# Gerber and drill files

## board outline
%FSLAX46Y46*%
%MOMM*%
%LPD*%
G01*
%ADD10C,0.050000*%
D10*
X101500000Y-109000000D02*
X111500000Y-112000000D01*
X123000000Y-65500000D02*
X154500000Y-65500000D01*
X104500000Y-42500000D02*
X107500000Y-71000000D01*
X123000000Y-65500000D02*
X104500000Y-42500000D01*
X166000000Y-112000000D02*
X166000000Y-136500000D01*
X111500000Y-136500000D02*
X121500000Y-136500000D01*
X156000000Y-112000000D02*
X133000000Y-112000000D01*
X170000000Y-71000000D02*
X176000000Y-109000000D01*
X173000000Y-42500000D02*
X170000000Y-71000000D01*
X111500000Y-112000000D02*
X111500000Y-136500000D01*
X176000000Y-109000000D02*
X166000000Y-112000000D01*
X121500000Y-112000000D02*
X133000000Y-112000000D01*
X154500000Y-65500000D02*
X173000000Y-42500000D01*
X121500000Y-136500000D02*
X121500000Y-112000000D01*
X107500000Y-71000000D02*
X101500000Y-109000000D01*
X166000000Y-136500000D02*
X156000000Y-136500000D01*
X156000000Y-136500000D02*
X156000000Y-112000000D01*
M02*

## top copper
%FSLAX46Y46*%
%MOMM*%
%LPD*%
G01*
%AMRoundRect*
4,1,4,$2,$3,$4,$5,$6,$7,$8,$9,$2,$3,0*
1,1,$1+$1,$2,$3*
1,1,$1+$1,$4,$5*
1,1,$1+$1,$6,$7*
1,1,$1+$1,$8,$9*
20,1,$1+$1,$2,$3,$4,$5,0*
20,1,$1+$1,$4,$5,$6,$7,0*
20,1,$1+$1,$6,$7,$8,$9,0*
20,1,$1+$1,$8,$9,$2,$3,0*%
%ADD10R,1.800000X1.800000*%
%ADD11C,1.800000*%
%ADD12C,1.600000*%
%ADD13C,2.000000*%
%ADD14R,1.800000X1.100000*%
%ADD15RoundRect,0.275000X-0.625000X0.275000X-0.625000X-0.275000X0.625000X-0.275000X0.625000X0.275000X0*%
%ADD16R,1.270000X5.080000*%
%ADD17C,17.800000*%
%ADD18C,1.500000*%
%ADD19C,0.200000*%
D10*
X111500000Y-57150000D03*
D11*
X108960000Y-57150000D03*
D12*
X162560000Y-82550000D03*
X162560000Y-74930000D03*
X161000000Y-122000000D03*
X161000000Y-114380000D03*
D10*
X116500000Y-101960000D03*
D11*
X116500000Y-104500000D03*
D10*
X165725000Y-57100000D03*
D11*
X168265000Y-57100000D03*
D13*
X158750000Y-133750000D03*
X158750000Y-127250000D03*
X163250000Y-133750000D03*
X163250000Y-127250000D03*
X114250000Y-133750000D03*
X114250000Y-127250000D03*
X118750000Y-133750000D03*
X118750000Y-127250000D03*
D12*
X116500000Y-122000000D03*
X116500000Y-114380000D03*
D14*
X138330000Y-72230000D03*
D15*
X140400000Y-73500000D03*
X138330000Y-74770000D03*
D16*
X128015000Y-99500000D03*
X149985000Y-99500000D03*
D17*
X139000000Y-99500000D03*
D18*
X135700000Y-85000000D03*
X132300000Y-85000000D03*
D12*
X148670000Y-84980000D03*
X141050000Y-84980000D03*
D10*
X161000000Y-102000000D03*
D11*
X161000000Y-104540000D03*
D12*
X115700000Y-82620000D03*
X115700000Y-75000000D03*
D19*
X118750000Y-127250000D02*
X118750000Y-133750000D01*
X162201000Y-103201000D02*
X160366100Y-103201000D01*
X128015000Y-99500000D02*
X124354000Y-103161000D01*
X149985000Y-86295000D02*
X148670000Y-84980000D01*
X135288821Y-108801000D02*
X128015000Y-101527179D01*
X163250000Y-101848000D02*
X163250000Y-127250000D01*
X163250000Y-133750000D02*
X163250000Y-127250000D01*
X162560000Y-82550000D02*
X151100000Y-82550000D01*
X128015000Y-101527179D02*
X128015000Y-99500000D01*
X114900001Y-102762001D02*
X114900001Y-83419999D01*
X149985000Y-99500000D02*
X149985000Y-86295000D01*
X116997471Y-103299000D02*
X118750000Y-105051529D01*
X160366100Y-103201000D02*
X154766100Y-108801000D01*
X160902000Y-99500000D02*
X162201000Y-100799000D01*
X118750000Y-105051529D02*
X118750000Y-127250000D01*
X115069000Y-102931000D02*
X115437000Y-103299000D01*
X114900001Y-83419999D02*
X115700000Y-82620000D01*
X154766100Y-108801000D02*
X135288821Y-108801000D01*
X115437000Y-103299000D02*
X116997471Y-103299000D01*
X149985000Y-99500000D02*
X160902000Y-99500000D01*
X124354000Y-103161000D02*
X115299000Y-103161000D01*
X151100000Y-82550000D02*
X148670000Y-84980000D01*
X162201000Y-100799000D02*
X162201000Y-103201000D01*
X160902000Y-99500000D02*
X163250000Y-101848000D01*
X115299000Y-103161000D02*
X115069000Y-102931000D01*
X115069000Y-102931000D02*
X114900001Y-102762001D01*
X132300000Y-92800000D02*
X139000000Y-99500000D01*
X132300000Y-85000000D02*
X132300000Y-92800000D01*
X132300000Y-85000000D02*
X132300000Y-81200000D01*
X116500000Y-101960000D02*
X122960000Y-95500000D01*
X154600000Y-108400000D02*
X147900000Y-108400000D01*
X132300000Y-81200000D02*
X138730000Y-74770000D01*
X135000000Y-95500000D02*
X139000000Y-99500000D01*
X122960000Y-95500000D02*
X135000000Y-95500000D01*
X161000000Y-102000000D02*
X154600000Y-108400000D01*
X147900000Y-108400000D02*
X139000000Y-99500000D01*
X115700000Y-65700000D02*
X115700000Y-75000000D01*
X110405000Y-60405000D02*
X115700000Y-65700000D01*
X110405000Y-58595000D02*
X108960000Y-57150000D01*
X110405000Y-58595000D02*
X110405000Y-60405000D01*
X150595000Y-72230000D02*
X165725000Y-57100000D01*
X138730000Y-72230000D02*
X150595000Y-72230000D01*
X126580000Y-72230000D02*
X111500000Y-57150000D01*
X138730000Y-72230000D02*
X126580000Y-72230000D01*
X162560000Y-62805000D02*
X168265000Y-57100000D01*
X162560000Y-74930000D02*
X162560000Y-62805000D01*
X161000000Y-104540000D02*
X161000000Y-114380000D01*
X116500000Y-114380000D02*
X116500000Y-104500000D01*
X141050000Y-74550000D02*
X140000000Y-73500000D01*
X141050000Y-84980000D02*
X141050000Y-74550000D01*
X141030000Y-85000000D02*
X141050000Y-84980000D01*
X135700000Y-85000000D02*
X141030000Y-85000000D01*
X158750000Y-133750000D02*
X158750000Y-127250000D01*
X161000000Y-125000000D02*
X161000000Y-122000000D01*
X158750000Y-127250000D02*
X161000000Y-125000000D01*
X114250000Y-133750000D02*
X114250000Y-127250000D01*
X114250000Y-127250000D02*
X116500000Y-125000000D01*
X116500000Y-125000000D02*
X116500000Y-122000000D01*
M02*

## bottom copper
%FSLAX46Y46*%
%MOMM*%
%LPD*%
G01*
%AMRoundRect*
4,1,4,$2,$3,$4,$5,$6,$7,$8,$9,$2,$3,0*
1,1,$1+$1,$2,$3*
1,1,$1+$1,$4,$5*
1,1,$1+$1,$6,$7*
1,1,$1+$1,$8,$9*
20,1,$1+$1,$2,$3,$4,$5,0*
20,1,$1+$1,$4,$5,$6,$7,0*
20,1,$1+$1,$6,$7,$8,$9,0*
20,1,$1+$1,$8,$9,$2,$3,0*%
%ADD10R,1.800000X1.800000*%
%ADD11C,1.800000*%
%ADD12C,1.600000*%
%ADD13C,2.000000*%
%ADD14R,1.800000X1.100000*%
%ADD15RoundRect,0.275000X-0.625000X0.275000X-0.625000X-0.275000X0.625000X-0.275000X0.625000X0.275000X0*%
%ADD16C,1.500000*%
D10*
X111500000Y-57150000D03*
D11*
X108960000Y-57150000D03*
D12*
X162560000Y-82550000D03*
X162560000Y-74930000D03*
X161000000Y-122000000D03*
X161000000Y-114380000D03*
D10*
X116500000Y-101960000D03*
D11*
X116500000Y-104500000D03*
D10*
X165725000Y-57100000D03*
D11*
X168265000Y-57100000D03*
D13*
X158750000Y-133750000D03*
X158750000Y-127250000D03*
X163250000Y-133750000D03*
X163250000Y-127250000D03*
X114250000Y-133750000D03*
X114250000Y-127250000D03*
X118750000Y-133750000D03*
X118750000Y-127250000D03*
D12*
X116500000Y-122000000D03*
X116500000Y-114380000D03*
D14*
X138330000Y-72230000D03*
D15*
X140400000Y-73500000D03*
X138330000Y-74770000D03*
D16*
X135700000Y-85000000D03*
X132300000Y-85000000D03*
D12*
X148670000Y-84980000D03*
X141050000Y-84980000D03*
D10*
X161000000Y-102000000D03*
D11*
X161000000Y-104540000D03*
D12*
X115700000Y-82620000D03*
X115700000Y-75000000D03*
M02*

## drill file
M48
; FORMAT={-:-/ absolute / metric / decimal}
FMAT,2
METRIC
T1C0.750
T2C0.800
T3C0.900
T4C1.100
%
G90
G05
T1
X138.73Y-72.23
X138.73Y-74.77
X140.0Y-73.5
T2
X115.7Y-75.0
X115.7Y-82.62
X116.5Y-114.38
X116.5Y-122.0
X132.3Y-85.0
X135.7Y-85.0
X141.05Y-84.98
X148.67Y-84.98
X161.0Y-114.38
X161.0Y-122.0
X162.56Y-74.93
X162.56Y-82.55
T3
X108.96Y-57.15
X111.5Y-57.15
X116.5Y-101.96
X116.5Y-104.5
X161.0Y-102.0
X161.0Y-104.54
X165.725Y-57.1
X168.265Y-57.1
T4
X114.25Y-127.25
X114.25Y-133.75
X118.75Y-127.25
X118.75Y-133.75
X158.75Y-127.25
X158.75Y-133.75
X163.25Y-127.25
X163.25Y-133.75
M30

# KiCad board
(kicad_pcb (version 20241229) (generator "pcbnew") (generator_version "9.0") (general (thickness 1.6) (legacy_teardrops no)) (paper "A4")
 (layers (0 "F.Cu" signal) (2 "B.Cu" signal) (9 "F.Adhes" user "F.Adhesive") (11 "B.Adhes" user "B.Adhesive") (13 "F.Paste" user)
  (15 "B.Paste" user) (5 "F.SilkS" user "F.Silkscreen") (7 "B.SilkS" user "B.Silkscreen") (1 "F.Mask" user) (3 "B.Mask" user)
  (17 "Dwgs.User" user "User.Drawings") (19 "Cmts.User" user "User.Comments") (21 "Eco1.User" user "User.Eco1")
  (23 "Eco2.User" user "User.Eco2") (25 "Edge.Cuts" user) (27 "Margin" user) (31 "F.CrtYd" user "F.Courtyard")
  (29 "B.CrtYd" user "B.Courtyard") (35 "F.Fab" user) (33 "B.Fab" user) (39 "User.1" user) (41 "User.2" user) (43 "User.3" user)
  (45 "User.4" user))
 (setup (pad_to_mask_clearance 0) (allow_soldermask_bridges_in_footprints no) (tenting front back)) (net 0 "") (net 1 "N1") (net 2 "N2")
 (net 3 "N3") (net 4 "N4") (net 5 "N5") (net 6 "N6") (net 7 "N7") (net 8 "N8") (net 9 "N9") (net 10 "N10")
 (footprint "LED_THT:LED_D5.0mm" (layer "F.Cu") (at 111.5 57.15 180)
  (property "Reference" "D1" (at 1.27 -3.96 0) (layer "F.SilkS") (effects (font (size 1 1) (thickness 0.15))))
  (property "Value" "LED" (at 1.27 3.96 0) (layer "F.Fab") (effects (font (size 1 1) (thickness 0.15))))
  (pad "1" thru_hole rect (at 0 0 180) (size 1.8 1.8) (drill 0.9) (layers "*.Cu" "*.Mask") (remove_unused_layers no) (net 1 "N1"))
  (pad "2" thru_hole circle (at 2.54 0 180) (size 1.8 1.8) (drill 0.9) (layers "*.Cu" "*.Mask") (remove_unused_layers no) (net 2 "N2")))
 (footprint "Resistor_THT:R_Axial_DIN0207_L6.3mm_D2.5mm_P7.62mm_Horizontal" (layer "F.Cu") (at 162.56 82.55 90)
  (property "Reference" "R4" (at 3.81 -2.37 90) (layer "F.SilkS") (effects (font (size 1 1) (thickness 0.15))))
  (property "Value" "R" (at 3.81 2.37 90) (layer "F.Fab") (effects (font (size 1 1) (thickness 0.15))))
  (pad "1" thru_hole circle (at 0 0 90) (size 1.6 1.6) (drill 0.8) (layers "*.Cu" "*.Mask") (remove_unused_layers no) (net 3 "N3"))
  (pad "2" thru_hole circle (at 7.62 0 90) (size 1.6 1.6) (drill 0.8) (layers "*.Cu" "*.Mask") (remove_unused_layers no) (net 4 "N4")))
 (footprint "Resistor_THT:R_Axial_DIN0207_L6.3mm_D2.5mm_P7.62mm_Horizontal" (layer "F.Cu") (at 161 122 90)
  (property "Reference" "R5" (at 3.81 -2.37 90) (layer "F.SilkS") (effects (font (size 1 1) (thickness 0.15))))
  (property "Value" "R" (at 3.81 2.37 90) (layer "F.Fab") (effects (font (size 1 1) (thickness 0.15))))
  (pad "1" thru_hole circle (at 0 0 90) (size 1.6 1.6) (drill 0.8) (layers "*.Cu" "*.Mask") (remove_unused_layers no) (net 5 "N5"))
  (pad "2" thru_hole circle (at 7.62 0 90) (size 1.6 1.6) (drill 0.8) (layers "*.Cu" "*.Mask") (remove_unused_layers no) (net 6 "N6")))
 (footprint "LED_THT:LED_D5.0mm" (layer "F.Cu") (at 116.5 101.96 -90)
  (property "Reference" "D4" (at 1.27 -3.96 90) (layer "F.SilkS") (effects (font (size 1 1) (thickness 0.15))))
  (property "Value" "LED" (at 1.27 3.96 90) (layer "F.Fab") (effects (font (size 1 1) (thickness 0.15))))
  (pad "1" thru_hole rect (at 0 0 270) (size 1.8 1.8) (drill 0.9) (layers "*.Cu" "*.Mask") (remove_unused_layers no) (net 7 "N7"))
  (pad "2" thru_hole circle (at 2.54 0 270) (size 1.8 1.8) (drill 0.9) (layers "*.Cu" "*.Mask") (remove_unused_layers no) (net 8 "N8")))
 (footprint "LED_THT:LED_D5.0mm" (layer "F.Cu") (at 165.725 57.1)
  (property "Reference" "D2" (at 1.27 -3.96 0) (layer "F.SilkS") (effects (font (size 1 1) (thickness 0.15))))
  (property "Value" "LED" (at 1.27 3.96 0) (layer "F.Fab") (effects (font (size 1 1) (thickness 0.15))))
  (pad "1" thru_hole rect (at 0 0) (size 1.8 1.8) (drill 0.9) (layers "*.Cu" "*.Mask") (remove_unused_layers no) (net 1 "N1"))
  (pad "2" thru_hole circle (at 2.54 0) (size 1.8 1.8) (drill 0.9) (layers "*.Cu" "*.Mask") (remove_unused_layers no) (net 4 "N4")))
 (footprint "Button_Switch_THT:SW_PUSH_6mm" (layer "F.Cu") (at 158.75 133.75 90)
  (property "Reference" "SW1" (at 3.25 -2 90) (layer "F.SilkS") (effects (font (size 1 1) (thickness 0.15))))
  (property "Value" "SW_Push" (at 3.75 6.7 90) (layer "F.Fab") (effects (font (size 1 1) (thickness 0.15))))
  (pad "1" thru_hole circle (at 0 0 180) (size 2 2) (drill 1.1) (layers "*.Cu" "*.Mask") (remove_unused_layers no) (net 5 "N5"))
  (pad "1" thru_hole circle (at 6.5 0 180) (size 2 2) (drill 1.1) (layers "*.Cu" "*.Mask") (remove_unused_layers no) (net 5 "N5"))
  (pad "2" thru_hole circle (at 0 4.5 180) (size 2 2) (drill 1.1) (layers "*.Cu" "*.Mask") (remove_unused_layers no) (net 3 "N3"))
  (pad "2" thru_hole circle (at 6.5 4.5 180) (size 2 2) (drill 1.1) (layers "*.Cu" "*.Mask") (remove_unused_layers no) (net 3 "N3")))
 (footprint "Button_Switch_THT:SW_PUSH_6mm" (layer "F.Cu") (at 114.25 133.75 90)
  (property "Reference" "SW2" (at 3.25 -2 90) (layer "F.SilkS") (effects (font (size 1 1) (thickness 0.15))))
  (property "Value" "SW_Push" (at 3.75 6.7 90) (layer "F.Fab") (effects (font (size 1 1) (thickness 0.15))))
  (pad "1" thru_hole circle (at 0 0 180) (size 2 2) (drill 1.1) (layers "*.Cu" "*.Mask") (remove_unused_layers no) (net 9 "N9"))
  (pad "1" thru_hole circle (at 6.5 0 180) (size 2 2) (drill 1.1) (layers "*.Cu" "*.Mask") (remove_unused_layers no) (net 9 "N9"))
  (pad "2" thru_hole circle (at 0 4.5 180) (size 2 2) (drill 1.1) (layers "*.Cu" "*.Mask") (remove_unused_layers no) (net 3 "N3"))
  (pad "2" thru_hole circle (at 6.5 4.5 180) (size 2 2) (drill 1.1) (layers "*.Cu" "*.Mask") (remove_unused_layers no) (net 3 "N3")))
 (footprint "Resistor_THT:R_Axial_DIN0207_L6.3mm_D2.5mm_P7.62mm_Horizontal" (layer "F.Cu") (at 116.5 122 90)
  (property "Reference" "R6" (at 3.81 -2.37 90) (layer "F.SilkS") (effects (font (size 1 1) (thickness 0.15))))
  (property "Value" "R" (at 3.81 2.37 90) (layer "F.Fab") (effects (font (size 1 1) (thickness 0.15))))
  (pad "1" thru_hole circle (at 0 0 90) (size 1.6 1.6) (drill 0.8) (layers "*.Cu" "*.Mask") (remove_unused_layers no) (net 9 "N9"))
  (pad "2" thru_hole circle (at 7.62 0 90) (size 1.6 1.6) (drill 0.8) (layers "*.Cu" "*.Mask") (remove_unused_layers no) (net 8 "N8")))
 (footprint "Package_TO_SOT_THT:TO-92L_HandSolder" (layer "F.Cu") (at 138.73 72.23 -90)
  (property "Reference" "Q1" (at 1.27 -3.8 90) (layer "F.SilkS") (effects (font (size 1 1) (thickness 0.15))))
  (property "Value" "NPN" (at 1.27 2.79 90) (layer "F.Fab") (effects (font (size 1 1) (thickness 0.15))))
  (pad "1" thru_hole rect (at 0 0 270) (size 1.1 1.8) (drill 0.75 (offset 0 0.4)) (layers "*.Cu" "*.Mask") (remove_unused_layers no)
   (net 1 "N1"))
  (pad "2" thru_hole roundrect (at 1.27 -1.27 270) (size 1.1 1.8) (drill 0.75 (offset 0 -0.4)) (layers "*.Cu" "*.Mask")
   (remove_unused_layers no) (roundrect_rratio 0.25) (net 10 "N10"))
  (pad "3" thru_hole roundrect (at 2.54 0 270) (size 1.1 1.8) (drill 0.75 (offset 0 0.4)) (layers "*.Cu" "*.Mask") (remove_unused_layers no)
   (roundrect_rratio 0.25) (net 7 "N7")))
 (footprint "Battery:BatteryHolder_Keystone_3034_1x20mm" (layer "F.Cu") (at 139 99.5)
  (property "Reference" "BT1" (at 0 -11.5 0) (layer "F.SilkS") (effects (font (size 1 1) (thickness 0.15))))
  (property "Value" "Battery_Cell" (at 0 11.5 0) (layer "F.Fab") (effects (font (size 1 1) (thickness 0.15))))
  (pad "1" smd rect (at -10.985 0) (size 1.27 5.08) (layers "F.Cu" "F.Mask" "F.Paste") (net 3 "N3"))
  (pad "1" smd rect (at 10.985 0) (size 1.27 5.08) (layers "F.Cu" "F.Mask" "F.Paste") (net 3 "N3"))
  (pad "2" smd circle (at 0 0) (size 17.8 17.8) (layers "F.Cu" "F.Mask") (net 7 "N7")))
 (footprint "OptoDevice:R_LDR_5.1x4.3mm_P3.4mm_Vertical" (layer "F.Cu") (at 135.7 85 180)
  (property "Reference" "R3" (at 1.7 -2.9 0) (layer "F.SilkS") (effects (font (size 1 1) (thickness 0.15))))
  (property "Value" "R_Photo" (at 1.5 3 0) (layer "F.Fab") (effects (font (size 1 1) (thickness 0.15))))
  (pad "1" thru_hole circle (at 0 0 180) (size 1.5 1.5) (drill 0.8) (layers "*.Cu" "*.Mask") (remove_unused_layers no) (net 10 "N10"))
  (pad "2" thru_hole circle (at 3.4 0 180) (size 1.5 1.5) (drill 0.8) (layers "*.Cu" "*.Mask") (remove_unused_layers no) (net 7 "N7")))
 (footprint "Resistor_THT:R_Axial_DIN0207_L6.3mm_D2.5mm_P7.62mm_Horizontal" (layer "F.Cu") (at 148.67 84.98 180)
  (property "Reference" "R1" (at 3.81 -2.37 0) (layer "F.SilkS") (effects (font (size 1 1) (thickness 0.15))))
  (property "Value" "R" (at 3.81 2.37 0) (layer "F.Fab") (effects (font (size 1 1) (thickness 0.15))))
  (pad "1" thru_hole circle (at 0 0 180) (size 1.6 1.6) (drill 0.8) (layers "*.Cu" "*.Mask") (remove_unused_layers no) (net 3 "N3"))
  (pad "2" thru_hole circle (at 7.62 0 180) (size 1.6 1.6) (drill 0.8) (layers "*.Cu" "*.Mask") (remove_unused_layers no) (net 10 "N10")))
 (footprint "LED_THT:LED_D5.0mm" (layer "F.Cu") (at 161 102 -90)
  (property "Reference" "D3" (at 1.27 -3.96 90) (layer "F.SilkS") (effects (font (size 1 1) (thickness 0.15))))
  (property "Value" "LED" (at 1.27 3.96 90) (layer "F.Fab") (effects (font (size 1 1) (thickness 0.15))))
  (pad "1" thru_hole rect (at 0 0 270) (size 1.8 1.8) (drill 0.9) (layers "*.Cu" "*.Mask") (remove_unused_layers no) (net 7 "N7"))
  (pad "2" thru_hole circle (at 2.54 0 270) (size 1.8 1.8) (drill 0.9) (layers "*.Cu" "*.Mask") (remove_unused_layers no) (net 6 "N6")))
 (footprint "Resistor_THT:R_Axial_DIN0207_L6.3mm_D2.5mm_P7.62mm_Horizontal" (layer "F.Cu") (at 115.7 82.62 90)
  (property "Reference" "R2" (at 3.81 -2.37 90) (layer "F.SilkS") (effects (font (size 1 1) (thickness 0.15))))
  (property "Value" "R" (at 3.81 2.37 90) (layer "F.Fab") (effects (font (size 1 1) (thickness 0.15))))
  (pad "1" thru_hole circle (at 0 0 90) (size 1.6 1.6) (drill 0.8) (layers "*.Cu" "*.Mask") (remove_unused_layers no) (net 3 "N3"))
  (pad "2" thru_hole circle (at 7.62 0 90) (size 1.6 1.6) (drill 0.8) (layers "*.Cu" "*.Mask") (remove_unused_layers no) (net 2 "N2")))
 (gr_line (start 101.5 109) (end 111.5 112) (stroke (width 0.05) (type default)) (layer "Edge.Cuts"))
 (gr_line (start 123 65.5) (end 154.5 65.5) (stroke (width 0.05) (type default)) (layer "Edge.Cuts"))
 (gr_line (start 104.5 42.5) (end 107.5 71) (stroke (width 0.05) (type default)) (layer "Edge.Cuts"))
 (gr_line (start 123 65.5) (end 104.5 42.5) (stroke (width 0.05) (type default)) (layer "Edge.Cuts"))
 (gr_line (start 166 112) (end 166 136.5) (stroke (width 0.05) (type default)) (layer "Edge.Cuts"))
 (gr_line (start 111.5 136.5) (end 121.5 136.5) (stroke (width 0.05) (type default)) (layer "Edge.Cuts"))
 (gr_line (start 156 112) (end 133 112) (stroke (width 0.05) (type default)) (layer "Edge.Cuts"))
 (gr_line (start 170 71) (end 176 109) (stroke (width 0.05) (type default)) (layer "Edge.Cuts"))
 (gr_line (start 173 42.5) (end 170 71) (stroke (width 0.05) (type default)) (layer "Edge.Cuts"))
 (gr_line (start 111.5 112) (end 111.5 136.5) (stroke (width 0.05) (type default)) (layer "Edge.Cuts"))
 (gr_line (start 176 109) (end 166 112) (stroke (width 0.05) (type default)) (layer "Edge.Cuts"))
 (gr_line (start 121.5 112) (end 133 112) (stroke (width 0.05) (type default)) (layer "Edge.Cuts"))
 (gr_line (start 154.5 65.5) (end 173 42.5) (stroke (width 0.05) (type default)) (layer "Edge.Cuts"))
 (gr_line (start 121.5 136.5) (end 121.5 112) (stroke (width 0.05) (type default)) (layer "Edge.Cuts"))
 (gr_line (start 107.5 71) (end 101.5 109) (stroke (width 0.05) (type default)) (layer "Edge.Cuts"))
 (gr_line (start 166 136.5) (end 156 136.5) (stroke (width 0.05) (type default)) (layer "Edge.Cuts"))
 (gr_line (start 156 136.5) (end 156 112) (stroke (width 0.05) (type default)) (layer "Edge.Cuts"))
 (segment (start 118.75 127.25) (end 118.75 133.75) (width 0.2) (layer "F.Cu") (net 3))
 (segment (start 162.201 103.201) (end 160.3661 103.201) (width 0.2) (layer "F.Cu") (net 3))
 (segment (start 128.015 99.5) (end 124.354 103.161) (width 0.2) (layer "F.Cu") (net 3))
 (segment (start 149.985 86.295) (end 148.67 84.98) (width 0.2) (layer "F.Cu") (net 3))
 (segment (start 135.288821 108.801) (end 128.015 101.527179) (width 0.2) (layer "F.Cu") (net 3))
 (segment (start 163.25 101.848) (end 163.25 127.25) (width 0.2) (layer "F.Cu") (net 3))
 (segment (start 163.25 133.75) (end 163.25 127.25) (width 0.2) (layer "F.Cu") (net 3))
 (segment (start 162.56 82.55) (end 151.1 82.55) (width 0.2) (layer "F.Cu") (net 3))
 (segment (start 128.015 101.527179) (end 128.015 99.5) (width 0.2) (layer "F.Cu") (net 3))
 (segment (start 114.900001 102.762001) (end 114.900001 83.419999) (width 0.2) (layer "F.Cu") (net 3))
 (segment (start 149.985 99.5) (end 149.985 86.295) (width 0.2) (layer "F.Cu") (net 3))
 (segment (start 116.997471 103.299) (end 118.75 105.051529) (width 0.2) (layer "F.Cu") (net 3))
 (segment (start 160.3661 103.201) (end 154.7661 108.801) (width 0.2) (layer "F.Cu") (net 3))
 (segment (start 160.902 99.5) (end 162.201 100.799) (width 0.2) (layer "F.Cu") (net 3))
 (segment (start 118.75 105.051529) (end 118.75 127.25) (width 0.2) (layer "F.Cu") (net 3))
 (segment (start 115.069 102.931) (end 115.437 103.299) (width 0.2) (layer "F.Cu") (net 3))
 (segment (start 114.900001 83.419999) (end 115.7 82.62) (width 0.2) (layer "F.Cu") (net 3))
 (segment (start 154.7661 108.801) (end 135.288821 108.801) (width 0.2) (layer "F.Cu") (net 3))
 (segment (start 115.437 103.299) (end 116.997471 103.299) (width 0.2) (layer "F.Cu") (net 3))
 (segment (start 149.985 99.5) (end 160.902 99.5) (width 0.2) (layer "F.Cu") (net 3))
 (segment (start 124.354 103.161) (end 115.299 103.161) (width 0.2) (layer "F.Cu") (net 3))
 (segment (start 151.1 82.55) (end 148.67 84.98) (width 0.2) (layer "F.Cu") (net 3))
 (segment (start 162.201 100.799) (end 162.201 103.201) (width 0.2) (layer "F.Cu") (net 3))
 (segment (start 160.902 99.5) (end 163.25 101.848) (width 0.2) (layer "F.Cu") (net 3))
 (segment (start 115.299 103.161) (end 115.069 102.931) (width 0.2) (layer "F.Cu") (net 3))
 (segment (start 115.069 102.931) (end 114.900001 102.762001) (width 0.2) (layer "F.Cu") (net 3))
 (segment (start 132.3 92.8) (end 139 99.5) (width 0.2) (layer "F.Cu") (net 7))
 (segment (start 132.3 85) (end 132.3 92.8) (width 0.2) (layer "F.Cu") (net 7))
 (segment (start 132.3 85) (end 132.3 81.2) (width 0.2) (layer "F.Cu") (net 7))
 (segment (start 116.5 101.96) (end 122.96 95.5) (width 0.2) (layer "F.Cu") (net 7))
 (segment (start 154.6 108.4) (end 147.9 108.4) (width 0.2) (layer "F.Cu") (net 7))
 (segment (start 132.3 81.2) (end 138.73 74.77) (width 0.2) (layer "F.Cu") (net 7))
 (segment (start 135 95.5) (end 139 99.5) (width 0.2) (layer "F.Cu") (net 7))
 (segment (start 122.96 95.5) (end 135 95.5) (width 0.2) (layer "F.Cu") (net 7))
 (segment (start 161 102) (end 154.6 108.4) (width 0.2) (layer "F.Cu") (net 7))
 (segment (start 147.9 108.4) (end 139 99.5) (width 0.2) (layer "F.Cu") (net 7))
 (segment (start 115.7 65.7) (end 115.7 75) (width 0.2) (layer "F.Cu") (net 2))
 (segment (start 110.405 60.405) (end 115.7 65.7) (width 0.2) (layer "F.Cu") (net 2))
 (segment (start 110.405 58.595) (end 108.96 57.15) (width 0.2) (layer "F.Cu") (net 2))
 (segment (start 110.405 58.595) (end 110.405 60.405) (width 0.2) (layer "F.Cu") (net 2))
 (segment (start 150.595 72.23) (end 165.725 57.1) (width 0.2) (layer "F.Cu") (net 1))
 (segment (start 138.73 72.23) (end 150.595 72.23) (width 0.2) (layer "F.Cu") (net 1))
 (segment (start 126.58 72.23) (end 111.5 57.15) (width 0.2) (layer "F.Cu") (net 1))
 (segment (start 138.73 72.23) (end 126.58 72.23) (width 0.2) (layer "F.Cu") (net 1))
 (segment (start 162.56 62.805) (end 168.265 57.1) (width 0.2) (layer "F.Cu") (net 4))
 (segment (start 162.56 74.93) (end 162.56 62.805) (width 0.2) (layer "F.Cu") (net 4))
 (segment (start 161 104.54) (end 161 114.38) (width 0.2) (layer "F.Cu") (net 6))
 (segment (start 116.5 114.38) (end 116.5 104.5) (width 0.2) (layer "F.Cu") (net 8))
 (segment (start 141.05 74.55) (end 140 73.5) (width 0.2) (layer "F.Cu") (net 10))
 (segment (start 141.05 84.98) (end 141.05 74.55) (width 0.2) (layer "F.Cu") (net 10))
 (segment (start 141.03 85) (end 141.05 84.98) (width 0.2) (layer "F.Cu") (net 10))
 (segment (start 135.7 85) (end 141.03 85) (width 0.2) (layer "F.Cu") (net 10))
 (segment (start 158.75 133.75) (end 158.75 127.25) (width 0.2) (layer "F.Cu") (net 5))
 (segment (start 161 125) (end 161 122) (width 0.2) (layer "F.Cu") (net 5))
 (segment (start 158.75 127.25) (end 161 125) (width 0.2) (layer "F.Cu") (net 5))
 (segment (start 114.25 133.75) (end 114.25 127.25) (width 0.2) (layer "F.Cu") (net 9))
 (segment (start 114.25 127.25) (end 116.5 125) (width 0.2) (layer "F.Cu") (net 9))
 (segment (start 116.5 125) (end 116.5 122) (width 0.2) (layer "F.Cu") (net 9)))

